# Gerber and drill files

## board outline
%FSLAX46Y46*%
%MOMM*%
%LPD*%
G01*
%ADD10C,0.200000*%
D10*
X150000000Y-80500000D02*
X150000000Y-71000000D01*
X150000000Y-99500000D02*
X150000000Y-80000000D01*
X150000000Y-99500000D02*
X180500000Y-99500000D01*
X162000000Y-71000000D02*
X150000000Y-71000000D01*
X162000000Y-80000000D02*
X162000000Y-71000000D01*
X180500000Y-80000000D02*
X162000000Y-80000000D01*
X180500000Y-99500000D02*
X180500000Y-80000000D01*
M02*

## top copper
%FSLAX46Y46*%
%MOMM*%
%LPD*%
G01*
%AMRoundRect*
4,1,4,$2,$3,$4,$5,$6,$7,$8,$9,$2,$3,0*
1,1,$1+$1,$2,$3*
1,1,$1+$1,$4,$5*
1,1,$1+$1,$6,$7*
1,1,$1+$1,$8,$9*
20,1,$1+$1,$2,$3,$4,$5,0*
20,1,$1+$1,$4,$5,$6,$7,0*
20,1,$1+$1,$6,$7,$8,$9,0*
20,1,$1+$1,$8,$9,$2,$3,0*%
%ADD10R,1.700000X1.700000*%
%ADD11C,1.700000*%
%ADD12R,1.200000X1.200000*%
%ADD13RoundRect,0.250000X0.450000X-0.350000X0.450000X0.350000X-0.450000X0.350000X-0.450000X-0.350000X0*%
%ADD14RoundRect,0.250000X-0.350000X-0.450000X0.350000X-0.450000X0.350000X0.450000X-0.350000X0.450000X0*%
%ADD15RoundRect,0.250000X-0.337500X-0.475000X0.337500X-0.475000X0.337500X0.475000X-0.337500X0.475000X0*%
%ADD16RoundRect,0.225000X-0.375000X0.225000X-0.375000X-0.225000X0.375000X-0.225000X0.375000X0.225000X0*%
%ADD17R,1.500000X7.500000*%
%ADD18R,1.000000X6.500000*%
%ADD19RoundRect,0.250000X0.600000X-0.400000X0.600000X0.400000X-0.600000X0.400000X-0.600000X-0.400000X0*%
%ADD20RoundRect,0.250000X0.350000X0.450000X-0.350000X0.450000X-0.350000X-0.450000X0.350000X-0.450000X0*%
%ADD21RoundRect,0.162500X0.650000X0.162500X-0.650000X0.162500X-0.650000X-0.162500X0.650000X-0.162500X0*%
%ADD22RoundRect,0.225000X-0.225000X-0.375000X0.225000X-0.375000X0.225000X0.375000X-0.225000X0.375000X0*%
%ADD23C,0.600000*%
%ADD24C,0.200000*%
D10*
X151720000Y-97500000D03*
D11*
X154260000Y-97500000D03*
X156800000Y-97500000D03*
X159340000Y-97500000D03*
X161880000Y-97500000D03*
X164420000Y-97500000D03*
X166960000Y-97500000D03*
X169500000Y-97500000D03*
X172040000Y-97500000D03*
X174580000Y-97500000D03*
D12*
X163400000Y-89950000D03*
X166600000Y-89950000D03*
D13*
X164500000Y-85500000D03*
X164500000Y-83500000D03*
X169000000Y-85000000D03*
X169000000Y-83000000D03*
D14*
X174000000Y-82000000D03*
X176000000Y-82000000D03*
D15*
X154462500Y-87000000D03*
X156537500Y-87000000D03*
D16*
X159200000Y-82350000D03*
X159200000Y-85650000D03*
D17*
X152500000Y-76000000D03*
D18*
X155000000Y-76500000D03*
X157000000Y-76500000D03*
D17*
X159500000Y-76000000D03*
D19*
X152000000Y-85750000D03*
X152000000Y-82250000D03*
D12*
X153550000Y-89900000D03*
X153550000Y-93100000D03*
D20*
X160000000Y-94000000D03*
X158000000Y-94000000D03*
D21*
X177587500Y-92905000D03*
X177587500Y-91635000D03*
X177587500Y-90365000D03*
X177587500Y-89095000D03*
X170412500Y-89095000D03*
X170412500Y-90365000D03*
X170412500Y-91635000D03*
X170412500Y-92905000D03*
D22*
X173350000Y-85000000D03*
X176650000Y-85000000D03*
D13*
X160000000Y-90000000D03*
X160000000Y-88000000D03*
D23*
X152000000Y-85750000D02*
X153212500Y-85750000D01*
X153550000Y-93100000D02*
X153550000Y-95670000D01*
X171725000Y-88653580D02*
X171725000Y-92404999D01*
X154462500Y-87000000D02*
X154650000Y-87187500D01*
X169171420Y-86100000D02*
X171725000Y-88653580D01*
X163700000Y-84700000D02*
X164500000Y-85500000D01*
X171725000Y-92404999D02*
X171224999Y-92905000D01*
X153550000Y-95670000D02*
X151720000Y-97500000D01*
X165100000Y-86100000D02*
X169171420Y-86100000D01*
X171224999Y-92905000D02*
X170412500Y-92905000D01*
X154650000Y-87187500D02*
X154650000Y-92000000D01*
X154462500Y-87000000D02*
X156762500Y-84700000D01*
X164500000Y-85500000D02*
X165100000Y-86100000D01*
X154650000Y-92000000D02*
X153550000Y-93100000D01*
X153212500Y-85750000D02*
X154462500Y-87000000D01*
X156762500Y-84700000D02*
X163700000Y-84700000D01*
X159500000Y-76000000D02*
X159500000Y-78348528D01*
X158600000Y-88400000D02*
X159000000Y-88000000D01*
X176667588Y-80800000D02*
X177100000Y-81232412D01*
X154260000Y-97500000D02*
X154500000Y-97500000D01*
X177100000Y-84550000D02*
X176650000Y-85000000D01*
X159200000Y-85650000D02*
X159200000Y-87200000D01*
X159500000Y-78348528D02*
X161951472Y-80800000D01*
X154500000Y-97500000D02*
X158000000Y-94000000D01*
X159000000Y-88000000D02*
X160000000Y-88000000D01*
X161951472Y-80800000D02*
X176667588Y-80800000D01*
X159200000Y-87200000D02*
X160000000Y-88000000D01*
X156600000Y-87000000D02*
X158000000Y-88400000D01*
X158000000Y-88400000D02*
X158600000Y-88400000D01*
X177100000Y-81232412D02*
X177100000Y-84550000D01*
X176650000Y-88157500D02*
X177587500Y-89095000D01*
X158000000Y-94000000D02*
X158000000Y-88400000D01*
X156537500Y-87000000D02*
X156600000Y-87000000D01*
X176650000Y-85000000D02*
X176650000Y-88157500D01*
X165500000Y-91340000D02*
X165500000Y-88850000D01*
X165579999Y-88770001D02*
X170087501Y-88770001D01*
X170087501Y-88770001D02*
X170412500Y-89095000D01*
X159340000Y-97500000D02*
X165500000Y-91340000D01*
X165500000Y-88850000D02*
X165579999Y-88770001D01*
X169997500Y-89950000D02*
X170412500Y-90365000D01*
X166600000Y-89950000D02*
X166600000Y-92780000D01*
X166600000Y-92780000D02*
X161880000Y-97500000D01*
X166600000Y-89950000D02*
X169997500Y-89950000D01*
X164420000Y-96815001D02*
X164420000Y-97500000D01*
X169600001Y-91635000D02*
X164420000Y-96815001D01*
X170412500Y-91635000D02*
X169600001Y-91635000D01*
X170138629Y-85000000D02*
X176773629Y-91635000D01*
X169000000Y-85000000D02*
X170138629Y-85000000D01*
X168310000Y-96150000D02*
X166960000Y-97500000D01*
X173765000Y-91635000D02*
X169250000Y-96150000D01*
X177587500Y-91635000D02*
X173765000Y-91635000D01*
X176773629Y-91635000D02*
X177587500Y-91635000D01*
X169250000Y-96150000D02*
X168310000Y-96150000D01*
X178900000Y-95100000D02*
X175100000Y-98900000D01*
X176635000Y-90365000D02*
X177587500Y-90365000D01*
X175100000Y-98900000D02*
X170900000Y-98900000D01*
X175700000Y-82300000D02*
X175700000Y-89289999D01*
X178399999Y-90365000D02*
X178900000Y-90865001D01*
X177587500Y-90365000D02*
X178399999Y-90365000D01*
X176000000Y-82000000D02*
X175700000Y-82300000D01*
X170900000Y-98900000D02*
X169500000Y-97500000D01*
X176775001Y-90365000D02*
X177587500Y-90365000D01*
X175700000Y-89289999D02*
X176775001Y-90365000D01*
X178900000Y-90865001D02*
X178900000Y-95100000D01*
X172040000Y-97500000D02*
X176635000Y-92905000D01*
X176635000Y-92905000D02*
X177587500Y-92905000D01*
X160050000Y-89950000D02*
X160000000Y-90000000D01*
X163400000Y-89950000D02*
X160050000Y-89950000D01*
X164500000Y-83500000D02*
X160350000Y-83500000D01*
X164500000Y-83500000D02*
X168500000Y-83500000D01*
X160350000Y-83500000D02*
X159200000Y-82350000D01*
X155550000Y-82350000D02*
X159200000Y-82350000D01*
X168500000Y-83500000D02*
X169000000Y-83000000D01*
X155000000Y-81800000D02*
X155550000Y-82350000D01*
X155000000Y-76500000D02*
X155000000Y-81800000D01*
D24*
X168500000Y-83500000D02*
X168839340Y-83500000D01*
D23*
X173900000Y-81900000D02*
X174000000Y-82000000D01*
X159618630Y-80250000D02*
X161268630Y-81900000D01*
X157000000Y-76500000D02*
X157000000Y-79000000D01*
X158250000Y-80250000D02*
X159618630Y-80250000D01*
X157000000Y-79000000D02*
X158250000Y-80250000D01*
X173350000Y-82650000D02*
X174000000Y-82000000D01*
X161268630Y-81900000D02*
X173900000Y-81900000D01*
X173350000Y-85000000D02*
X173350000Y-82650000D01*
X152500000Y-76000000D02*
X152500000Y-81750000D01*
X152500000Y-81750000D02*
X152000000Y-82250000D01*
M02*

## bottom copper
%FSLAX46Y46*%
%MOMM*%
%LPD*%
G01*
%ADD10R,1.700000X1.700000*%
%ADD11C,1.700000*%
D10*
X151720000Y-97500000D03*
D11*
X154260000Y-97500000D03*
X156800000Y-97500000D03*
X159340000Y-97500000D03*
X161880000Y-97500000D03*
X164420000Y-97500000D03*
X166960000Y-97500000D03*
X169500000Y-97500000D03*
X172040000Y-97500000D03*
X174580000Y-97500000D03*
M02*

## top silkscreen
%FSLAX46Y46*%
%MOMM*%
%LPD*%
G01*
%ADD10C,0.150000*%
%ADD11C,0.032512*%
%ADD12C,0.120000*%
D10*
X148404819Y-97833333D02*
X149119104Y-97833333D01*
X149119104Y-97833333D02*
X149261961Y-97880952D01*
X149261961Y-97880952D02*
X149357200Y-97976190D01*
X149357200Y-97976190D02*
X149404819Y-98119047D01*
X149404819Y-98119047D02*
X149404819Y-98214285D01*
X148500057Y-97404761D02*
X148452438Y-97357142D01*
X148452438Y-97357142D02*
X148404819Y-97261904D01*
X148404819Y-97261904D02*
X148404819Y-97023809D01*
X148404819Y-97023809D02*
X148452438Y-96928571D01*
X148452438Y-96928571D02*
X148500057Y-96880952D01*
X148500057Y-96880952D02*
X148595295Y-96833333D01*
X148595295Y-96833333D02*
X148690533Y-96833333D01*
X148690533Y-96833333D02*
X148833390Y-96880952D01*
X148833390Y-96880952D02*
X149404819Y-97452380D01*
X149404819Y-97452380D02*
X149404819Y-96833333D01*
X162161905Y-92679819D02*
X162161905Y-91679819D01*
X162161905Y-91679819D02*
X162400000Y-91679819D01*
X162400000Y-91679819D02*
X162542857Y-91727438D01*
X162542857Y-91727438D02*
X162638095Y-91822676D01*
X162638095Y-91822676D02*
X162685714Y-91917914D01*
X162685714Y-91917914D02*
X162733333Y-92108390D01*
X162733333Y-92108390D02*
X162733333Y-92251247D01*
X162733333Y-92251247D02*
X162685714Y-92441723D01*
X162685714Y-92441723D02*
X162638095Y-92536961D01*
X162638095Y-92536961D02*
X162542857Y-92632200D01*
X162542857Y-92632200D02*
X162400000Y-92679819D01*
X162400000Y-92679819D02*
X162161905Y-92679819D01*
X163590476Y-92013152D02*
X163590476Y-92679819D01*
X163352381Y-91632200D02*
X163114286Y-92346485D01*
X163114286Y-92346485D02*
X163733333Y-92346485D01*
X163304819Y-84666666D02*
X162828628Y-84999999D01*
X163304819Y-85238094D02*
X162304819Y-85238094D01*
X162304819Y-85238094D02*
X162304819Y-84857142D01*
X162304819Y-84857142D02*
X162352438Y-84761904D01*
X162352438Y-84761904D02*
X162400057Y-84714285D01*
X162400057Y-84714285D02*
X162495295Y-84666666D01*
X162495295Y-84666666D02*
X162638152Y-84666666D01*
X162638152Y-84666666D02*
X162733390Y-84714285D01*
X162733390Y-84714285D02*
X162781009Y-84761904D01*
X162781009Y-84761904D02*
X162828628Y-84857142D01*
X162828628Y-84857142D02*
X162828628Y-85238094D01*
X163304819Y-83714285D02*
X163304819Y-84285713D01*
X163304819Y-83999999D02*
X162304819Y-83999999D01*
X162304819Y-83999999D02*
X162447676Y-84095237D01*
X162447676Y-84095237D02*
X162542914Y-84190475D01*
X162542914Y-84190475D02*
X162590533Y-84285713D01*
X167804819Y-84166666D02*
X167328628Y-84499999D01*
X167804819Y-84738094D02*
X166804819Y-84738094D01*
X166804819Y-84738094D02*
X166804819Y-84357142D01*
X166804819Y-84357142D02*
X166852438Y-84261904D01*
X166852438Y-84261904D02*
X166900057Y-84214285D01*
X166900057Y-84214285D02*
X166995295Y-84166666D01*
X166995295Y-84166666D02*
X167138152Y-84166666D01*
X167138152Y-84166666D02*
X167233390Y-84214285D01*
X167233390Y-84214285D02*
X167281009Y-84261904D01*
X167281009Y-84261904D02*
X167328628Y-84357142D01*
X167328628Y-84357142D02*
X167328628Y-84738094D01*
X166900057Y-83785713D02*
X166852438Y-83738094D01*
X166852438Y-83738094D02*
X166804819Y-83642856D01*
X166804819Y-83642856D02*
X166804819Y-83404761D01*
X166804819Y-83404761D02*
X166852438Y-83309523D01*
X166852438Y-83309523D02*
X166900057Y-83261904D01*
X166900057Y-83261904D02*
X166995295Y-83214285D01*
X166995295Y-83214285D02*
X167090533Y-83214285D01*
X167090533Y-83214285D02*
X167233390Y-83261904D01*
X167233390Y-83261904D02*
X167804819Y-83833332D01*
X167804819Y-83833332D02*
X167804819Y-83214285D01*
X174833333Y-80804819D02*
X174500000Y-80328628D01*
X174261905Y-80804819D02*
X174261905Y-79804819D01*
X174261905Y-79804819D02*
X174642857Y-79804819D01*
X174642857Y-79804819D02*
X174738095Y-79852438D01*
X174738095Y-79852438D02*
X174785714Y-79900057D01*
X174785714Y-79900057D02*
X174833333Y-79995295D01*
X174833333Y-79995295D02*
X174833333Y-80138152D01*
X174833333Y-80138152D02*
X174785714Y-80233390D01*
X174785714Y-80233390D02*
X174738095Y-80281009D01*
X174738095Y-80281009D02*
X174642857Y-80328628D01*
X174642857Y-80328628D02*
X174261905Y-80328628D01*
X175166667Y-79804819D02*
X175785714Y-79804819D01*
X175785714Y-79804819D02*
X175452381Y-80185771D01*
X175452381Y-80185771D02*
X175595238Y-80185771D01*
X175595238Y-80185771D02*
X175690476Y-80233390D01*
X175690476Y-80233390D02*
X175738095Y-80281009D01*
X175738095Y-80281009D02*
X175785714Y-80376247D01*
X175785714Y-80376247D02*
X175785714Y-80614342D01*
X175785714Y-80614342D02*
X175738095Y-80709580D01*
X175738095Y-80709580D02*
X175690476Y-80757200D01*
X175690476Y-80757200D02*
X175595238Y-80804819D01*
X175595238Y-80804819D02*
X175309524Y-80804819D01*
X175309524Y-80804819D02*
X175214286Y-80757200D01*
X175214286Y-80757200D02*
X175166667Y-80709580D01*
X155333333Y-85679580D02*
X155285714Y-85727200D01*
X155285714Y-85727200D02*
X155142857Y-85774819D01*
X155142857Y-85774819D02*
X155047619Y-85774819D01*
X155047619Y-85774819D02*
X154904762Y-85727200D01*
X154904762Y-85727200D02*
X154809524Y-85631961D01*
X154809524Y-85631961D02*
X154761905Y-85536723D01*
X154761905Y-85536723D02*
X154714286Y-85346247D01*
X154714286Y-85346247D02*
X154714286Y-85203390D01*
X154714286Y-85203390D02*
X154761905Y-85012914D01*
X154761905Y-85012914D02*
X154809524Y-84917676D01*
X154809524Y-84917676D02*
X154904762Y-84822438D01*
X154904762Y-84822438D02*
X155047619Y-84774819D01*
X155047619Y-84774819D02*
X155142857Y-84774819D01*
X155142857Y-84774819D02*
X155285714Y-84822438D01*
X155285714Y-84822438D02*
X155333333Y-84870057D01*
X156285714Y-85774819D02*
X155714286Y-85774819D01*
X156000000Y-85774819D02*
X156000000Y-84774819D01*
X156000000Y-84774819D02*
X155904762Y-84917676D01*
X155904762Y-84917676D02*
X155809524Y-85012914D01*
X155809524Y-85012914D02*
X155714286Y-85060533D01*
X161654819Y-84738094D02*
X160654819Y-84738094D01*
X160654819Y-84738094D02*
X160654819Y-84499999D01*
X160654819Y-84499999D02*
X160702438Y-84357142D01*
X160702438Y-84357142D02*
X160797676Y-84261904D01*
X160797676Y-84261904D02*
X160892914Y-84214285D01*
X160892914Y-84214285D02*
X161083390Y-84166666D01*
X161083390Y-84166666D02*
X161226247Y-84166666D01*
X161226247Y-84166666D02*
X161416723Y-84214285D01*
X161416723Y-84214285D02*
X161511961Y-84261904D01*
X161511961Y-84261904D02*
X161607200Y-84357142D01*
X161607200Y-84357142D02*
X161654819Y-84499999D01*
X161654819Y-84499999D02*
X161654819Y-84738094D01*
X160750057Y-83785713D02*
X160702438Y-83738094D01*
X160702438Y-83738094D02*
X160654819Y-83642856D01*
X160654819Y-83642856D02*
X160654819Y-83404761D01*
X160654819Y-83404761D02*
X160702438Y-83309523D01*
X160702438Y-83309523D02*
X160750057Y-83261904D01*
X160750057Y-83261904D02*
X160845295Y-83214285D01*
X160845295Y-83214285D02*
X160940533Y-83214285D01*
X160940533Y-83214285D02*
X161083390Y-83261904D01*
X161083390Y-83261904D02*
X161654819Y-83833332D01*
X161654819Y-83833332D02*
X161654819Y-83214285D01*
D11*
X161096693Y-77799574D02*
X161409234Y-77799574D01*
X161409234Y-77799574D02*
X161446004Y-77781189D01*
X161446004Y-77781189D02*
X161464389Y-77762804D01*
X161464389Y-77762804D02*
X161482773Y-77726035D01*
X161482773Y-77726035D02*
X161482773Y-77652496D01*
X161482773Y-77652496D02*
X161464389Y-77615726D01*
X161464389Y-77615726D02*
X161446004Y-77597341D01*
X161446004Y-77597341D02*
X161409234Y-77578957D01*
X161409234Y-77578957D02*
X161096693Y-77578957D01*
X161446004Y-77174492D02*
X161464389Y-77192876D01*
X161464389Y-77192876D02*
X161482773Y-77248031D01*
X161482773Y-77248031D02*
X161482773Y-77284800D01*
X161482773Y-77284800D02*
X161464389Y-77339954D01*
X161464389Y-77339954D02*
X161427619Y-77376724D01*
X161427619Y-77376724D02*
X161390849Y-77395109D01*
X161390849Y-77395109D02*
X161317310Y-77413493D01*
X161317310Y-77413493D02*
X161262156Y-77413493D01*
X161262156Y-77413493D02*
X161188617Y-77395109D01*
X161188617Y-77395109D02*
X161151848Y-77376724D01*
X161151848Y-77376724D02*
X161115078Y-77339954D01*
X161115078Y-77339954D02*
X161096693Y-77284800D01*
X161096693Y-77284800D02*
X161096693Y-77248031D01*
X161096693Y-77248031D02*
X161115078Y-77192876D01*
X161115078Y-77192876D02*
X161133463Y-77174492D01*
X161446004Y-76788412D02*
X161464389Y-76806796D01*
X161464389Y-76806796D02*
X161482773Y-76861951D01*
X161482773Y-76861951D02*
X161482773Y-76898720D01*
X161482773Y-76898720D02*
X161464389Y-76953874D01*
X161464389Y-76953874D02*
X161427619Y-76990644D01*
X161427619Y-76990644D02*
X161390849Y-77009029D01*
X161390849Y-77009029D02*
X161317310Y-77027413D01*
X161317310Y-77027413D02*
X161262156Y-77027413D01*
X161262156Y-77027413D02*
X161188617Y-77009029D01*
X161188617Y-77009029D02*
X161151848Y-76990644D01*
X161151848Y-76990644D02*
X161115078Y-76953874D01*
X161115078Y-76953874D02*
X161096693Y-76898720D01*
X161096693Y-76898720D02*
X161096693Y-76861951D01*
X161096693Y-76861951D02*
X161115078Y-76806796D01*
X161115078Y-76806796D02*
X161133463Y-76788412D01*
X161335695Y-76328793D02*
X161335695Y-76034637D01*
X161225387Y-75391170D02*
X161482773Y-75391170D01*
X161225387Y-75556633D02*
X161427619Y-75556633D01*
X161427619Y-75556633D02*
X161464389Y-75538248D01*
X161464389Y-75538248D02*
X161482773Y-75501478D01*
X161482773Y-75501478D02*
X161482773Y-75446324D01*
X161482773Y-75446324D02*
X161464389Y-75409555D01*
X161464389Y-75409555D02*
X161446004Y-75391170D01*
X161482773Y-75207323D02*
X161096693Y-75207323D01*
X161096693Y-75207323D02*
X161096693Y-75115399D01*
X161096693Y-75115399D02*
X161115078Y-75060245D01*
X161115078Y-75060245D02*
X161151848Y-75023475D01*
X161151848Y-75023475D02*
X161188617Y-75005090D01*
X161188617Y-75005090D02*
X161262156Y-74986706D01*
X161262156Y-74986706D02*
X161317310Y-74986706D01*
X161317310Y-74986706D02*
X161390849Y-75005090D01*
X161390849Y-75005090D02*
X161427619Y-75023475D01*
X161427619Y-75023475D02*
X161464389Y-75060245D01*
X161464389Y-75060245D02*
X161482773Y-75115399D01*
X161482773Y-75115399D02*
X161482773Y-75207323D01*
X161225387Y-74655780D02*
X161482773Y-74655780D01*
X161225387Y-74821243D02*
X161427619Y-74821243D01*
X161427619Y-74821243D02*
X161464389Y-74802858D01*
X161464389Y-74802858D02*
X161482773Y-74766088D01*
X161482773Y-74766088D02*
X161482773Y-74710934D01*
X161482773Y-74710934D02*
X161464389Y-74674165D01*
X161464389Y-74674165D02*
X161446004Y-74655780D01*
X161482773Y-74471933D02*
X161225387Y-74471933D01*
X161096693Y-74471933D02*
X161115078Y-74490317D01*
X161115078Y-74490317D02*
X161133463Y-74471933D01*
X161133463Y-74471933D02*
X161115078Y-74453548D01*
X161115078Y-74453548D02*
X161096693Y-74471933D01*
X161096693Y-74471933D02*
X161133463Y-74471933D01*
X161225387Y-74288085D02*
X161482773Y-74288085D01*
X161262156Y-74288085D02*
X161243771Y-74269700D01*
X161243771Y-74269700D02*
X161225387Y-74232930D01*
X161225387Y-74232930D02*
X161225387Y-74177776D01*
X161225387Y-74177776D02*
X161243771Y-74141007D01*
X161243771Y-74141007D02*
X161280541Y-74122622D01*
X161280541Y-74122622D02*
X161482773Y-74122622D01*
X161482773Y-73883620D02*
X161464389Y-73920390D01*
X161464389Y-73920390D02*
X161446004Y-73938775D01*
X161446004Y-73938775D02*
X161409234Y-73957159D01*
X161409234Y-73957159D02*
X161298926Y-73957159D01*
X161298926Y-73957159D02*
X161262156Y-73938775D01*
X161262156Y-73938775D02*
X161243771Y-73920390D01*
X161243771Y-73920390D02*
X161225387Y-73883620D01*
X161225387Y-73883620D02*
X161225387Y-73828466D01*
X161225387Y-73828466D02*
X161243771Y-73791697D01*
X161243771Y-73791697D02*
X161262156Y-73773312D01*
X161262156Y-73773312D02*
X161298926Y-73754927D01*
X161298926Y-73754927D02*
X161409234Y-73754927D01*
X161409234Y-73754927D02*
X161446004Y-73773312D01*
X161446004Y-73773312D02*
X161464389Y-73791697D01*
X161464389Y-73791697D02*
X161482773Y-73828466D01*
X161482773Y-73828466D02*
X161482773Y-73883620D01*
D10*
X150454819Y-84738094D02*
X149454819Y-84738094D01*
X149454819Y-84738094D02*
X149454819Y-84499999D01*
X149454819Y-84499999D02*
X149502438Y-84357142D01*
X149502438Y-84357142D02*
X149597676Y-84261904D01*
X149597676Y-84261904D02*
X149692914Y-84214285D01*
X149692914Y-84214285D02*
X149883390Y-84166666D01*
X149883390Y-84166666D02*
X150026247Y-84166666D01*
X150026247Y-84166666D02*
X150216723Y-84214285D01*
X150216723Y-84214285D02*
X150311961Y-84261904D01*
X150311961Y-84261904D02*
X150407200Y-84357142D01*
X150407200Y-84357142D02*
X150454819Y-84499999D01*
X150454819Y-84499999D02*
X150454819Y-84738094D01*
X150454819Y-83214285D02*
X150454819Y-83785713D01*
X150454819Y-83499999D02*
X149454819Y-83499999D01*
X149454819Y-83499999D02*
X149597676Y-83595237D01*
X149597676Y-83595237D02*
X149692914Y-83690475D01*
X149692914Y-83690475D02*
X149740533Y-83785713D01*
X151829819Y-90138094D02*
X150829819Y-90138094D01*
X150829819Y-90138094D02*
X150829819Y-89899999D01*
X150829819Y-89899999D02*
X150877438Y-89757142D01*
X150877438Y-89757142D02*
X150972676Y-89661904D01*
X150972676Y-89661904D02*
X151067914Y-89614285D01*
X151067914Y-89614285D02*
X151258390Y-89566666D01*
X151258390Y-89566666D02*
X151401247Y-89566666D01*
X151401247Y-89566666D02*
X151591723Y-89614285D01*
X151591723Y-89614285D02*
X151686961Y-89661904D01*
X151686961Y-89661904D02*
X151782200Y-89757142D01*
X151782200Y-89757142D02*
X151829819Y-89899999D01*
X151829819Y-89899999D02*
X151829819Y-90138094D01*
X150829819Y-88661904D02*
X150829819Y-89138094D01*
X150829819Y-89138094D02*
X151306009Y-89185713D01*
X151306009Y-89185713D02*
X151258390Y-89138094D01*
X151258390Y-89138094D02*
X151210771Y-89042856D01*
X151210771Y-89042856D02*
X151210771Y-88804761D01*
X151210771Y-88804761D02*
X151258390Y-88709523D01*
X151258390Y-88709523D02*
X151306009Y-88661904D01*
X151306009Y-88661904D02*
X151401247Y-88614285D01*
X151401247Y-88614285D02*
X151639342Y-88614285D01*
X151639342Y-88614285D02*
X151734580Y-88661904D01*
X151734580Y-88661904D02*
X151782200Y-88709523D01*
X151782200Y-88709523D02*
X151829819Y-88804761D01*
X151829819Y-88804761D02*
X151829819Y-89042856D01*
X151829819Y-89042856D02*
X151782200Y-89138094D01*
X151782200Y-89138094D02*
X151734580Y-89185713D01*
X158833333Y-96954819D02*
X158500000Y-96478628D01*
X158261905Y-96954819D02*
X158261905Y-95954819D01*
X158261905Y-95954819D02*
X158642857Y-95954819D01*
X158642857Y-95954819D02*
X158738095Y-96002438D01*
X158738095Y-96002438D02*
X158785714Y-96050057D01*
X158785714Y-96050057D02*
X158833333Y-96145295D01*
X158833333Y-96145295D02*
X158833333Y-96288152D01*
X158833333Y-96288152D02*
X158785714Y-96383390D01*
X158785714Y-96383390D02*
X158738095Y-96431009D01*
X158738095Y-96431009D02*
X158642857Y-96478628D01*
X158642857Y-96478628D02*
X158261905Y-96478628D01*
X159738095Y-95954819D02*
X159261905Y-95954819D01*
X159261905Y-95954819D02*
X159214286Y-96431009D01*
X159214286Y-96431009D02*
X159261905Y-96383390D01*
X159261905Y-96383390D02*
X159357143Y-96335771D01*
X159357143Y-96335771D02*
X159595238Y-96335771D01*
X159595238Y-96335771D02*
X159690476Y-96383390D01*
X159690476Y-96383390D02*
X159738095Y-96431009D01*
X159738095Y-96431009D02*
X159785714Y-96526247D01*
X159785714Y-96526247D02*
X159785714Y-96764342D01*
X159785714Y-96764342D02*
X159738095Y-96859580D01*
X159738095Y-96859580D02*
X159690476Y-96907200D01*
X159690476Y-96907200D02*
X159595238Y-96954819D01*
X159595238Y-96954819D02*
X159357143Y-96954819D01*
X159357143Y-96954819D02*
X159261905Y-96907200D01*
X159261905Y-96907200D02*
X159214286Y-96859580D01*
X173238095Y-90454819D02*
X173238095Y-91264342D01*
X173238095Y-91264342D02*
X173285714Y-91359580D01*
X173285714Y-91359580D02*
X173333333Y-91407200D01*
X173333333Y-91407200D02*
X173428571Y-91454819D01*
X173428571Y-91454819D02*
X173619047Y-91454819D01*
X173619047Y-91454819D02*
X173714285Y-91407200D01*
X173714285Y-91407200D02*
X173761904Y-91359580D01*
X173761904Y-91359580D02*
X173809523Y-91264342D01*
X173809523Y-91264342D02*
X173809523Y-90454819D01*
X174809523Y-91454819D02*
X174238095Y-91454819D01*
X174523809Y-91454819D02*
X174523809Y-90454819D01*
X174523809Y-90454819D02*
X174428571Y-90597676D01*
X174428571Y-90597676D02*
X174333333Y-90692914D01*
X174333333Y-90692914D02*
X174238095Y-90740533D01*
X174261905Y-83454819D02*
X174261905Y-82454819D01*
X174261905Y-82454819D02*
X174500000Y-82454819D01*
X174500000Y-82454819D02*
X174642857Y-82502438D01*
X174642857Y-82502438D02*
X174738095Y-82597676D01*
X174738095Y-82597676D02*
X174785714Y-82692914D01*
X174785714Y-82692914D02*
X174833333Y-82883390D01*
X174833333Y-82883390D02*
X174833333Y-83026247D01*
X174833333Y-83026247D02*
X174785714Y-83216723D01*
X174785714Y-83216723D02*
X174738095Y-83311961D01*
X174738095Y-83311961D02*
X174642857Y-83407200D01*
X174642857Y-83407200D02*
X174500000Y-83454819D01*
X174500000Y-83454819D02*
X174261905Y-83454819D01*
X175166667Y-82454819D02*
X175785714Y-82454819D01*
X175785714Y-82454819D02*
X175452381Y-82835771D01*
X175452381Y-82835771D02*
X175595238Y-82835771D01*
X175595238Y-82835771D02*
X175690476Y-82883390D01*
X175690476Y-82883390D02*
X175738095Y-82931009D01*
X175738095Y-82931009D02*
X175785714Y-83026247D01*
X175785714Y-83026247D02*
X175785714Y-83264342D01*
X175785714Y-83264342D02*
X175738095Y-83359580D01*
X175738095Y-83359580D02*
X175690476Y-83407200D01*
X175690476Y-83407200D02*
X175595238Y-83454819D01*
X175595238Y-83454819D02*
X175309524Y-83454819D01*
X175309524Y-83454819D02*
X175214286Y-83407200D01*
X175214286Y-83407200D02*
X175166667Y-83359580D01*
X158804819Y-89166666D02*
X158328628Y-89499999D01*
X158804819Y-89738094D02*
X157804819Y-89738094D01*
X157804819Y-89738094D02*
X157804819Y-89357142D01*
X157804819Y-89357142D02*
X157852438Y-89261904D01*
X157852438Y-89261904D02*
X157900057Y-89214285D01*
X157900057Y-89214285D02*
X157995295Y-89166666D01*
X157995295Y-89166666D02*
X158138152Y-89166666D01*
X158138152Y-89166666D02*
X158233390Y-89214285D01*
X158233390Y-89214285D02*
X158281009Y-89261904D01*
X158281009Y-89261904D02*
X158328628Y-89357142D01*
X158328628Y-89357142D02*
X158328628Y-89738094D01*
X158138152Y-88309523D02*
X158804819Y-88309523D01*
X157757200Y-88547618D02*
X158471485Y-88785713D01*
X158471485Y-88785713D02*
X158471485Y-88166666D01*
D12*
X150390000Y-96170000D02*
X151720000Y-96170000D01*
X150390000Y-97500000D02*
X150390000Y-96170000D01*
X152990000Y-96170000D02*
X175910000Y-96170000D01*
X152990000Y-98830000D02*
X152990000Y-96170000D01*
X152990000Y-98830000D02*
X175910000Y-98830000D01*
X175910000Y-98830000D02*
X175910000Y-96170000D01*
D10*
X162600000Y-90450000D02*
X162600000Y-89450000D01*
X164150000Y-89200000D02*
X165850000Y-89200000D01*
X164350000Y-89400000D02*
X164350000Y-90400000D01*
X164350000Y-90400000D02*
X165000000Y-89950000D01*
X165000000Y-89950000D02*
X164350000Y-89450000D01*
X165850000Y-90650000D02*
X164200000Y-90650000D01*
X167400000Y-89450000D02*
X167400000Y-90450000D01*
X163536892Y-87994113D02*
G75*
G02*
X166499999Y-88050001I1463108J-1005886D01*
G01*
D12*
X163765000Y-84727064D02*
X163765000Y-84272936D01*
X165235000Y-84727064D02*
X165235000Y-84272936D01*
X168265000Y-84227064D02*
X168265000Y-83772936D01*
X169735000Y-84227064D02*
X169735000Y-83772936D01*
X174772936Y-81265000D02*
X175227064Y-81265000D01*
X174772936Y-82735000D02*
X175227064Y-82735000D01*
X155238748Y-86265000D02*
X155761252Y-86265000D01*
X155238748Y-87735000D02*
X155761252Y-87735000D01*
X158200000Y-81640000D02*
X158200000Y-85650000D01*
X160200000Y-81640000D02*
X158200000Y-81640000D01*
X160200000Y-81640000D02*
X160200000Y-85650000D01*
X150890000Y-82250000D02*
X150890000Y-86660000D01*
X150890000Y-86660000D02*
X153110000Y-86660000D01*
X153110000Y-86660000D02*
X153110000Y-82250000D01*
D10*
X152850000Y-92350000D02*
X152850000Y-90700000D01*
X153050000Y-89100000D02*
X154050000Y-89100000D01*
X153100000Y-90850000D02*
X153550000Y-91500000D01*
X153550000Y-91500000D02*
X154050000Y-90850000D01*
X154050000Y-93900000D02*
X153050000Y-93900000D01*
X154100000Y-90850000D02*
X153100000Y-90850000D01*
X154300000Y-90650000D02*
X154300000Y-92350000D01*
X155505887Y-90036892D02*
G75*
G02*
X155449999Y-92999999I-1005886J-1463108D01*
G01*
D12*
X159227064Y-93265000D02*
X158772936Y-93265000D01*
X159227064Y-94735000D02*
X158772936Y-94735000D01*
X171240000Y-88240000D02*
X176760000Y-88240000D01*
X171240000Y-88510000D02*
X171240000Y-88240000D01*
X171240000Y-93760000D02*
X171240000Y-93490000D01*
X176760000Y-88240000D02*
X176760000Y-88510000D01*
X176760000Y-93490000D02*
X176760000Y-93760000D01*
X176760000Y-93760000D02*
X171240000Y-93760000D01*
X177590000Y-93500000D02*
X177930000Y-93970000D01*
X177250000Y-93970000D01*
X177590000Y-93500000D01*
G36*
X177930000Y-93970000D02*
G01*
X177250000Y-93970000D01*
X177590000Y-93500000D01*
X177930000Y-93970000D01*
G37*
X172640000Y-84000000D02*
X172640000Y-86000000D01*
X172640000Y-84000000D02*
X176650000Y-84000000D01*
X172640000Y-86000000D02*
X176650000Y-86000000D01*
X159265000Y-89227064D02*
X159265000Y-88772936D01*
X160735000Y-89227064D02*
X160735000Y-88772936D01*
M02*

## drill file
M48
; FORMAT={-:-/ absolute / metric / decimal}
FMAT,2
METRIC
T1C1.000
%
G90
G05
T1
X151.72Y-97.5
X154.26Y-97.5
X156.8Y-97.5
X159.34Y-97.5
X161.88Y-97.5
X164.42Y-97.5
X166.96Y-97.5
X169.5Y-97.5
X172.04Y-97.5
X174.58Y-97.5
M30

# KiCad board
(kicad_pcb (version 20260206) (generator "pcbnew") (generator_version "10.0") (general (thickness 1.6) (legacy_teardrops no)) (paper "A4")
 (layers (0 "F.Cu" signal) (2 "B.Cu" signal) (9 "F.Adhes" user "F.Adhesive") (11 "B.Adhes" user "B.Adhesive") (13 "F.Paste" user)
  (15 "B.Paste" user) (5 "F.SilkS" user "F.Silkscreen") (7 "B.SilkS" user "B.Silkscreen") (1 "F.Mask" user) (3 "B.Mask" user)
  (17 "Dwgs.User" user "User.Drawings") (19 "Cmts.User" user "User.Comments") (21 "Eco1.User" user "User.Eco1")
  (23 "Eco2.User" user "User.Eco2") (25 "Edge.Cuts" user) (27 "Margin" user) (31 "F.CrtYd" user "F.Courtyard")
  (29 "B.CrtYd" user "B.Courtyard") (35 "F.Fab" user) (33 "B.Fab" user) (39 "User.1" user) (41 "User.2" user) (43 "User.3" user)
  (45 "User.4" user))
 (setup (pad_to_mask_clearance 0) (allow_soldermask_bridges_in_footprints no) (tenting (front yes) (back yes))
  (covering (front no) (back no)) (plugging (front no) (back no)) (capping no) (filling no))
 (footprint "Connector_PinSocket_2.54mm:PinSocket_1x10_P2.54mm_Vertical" (layer "F.Cu") (at 151.72 97.5 90)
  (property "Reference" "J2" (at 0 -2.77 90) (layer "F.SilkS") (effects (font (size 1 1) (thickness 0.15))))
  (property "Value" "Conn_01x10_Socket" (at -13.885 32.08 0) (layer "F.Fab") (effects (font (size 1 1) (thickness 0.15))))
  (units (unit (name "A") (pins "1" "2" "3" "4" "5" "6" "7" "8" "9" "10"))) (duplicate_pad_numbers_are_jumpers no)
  (fp_line (start 1.33 -1.33) (end 1.33 0) (stroke (width 0.12) (type solid)) (layer "F.SilkS"))
  (fp_line (start 0 -1.33) (end 1.33 -1.33) (stroke (width 0.12) (type solid)) (layer "F.SilkS"))
  (fp_line (start 1.33 1.27) (end 1.33 24.19) (stroke (width 0.12) (type solid)) (layer "F.SilkS"))
  (fp_line (start -1.33 1.27) (end 1.33 1.27) (stroke (width 0.12) (type solid)) (layer "F.SilkS"))
  (fp_line (start -1.33 1.27) (end -1.33 24.19) (stroke (width 0.12) (type solid)) (layer "F.SilkS"))
  (fp_line (start -1.33 24.19) (end 1.33 24.19) (stroke (width 0.12) (type solid)) (layer "F.SilkS"))
  (pad "1" thru_hole rect (at 0 0 90) (size 1.7 1.7) (drill 1) (layers "*.Cu" "*.Mask") (remove_unused_layers no) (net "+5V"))
  (pad "2" thru_hole circle (at 0 2.54 90) (size 1.7 1.7) (drill 1) (layers "*.Cu" "*.Mask") (remove_unused_layers no) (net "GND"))
  (pad "3" thru_hole circle (at 0 5.08 90) (size 1.7 1.7) (drill 1) (layers "*.Cu" "*.Mask") (remove_unused_layers no)
   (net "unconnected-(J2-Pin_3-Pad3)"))
  (pad "4" thru_hole circle (at 0 7.62 90) (size 1.7 1.7) (drill 1) (layers "*.Cu" "*.Mask") (remove_unused_layers no)
   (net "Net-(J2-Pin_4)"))
  (pad "5" thru_hole circle (at 0 10.16 90) (size 1.7 1.7) (drill 1) (layers "*.Cu" "*.Mask") (remove_unused_layers no) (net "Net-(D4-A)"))
  (pad "6" thru_hole circle (at 0 12.7 90) (size 1.7 1.7) (drill 1) (layers "*.Cu" "*.Mask") (remove_unused_layers no)
   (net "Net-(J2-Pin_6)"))
  (pad "7" thru_hole circle (at 0 15.24 90) (size 1.7 1.7) (drill 1) (layers "*.Cu" "*.Mask") (remove_unused_layers no)
   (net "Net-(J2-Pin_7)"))
  (pad "8" thru_hole circle (at 0 17.78 90) (size 1.7 1.7) (drill 1) (layers "*.Cu" "*.Mask") (remove_unused_layers no)
   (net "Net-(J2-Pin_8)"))
  (pad "9" thru_hole circle (at 0 20.32 90) (size 1.7 1.7) (drill 1) (layers "*.Cu" "*.Mask") (remove_unused_layers no)
   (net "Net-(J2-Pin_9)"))
  (pad "10" thru_hole circle (at 0 22.86 90) (size 1.7 1.7) (drill 1) (layers "*.Cu" "*.Mask") (remove_unused_layers no)
   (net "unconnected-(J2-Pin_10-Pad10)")))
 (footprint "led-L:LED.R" (layer "F.Cu") (at 165.5 89.5)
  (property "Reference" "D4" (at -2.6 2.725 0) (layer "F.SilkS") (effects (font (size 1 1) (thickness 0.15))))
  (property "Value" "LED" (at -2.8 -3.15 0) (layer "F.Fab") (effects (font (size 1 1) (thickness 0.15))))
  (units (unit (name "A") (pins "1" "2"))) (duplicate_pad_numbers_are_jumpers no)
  (fp_line (start -2.9 0.95) (end -2.9 -0.05) (stroke (width 0.15) (type solid)) (layer "F.SilkS"))
  (fp_line (start -1.35 -0.3) (end 0.35 -0.3) (stroke (width 0.15) (type solid)) (layer "F.SilkS"))
  (fp_line (start -1.15 -0.1) (end -1.15 0.9) (stroke (width 0.15) (type solid)) (layer "F.SilkS"))
  (fp_line (start -1.15 0.9) (end -0.5 0.45) (stroke (width 0.15) (type solid)) (layer "F.SilkS"))
  (fp_line (start -0.5 0.45) (end -1.15 -0.05) (stroke (width 0.15) (type solid)) (layer "F.SilkS"))
  (fp_line (start 0.35 1.15) (end -1.3 1.15) (stroke (width 0.15) (type solid)) (layer "F.SilkS"))
  (fp_line (start 1.9 -0.05) (end 1.9 0.95) (stroke (width 0.15) (type solid)) (layer "F.SilkS"))
  (fp_arc (start -1.963108 -1.505887) (mid -0.466517 -2.275211) (end 0.999999 -1.449999) (stroke (width 0.15) (type solid))
   (layer "F.SilkS"))
  (pad "1" smd rect (at -2.1 0.45) (size 1.2 1.2) (layers "F.Cu" "F.Mask" "F.Paste") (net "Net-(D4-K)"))
  (pad "2" smd rect (at 1.1 0.45) (size 1.2 1.2) (layers "F.Cu" "F.Mask" "F.Paste") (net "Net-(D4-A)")))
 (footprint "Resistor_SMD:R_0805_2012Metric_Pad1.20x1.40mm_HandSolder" (layer "F.Cu") (at 164.5 84.5 90)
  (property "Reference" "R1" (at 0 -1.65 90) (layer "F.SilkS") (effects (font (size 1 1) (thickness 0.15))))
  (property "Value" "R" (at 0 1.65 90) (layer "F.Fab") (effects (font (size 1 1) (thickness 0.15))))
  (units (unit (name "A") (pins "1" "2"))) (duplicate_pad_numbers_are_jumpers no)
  (fp_line (start -0.227064 -0.735) (end 0.227064 -0.735) (stroke (width 0.12) (type solid)) (layer "F.SilkS"))
  (fp_line (start -0.227064 0.735) (end 0.227064 0.735) (stroke (width 0.12) (type solid)) (layer "F.SilkS"))
  (pad "1" smd roundrect (at -1 0 90) (size 1.2 1.4) (layers "F.Cu" "F.Mask" "F.Paste") (roundrect_rratio 0.208333) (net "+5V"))
  (pad "2" smd roundrect (at 1 0 90) (size 1.2 1.4) (layers "F.Cu" "F.Mask" "F.Paste") (roundrect_rratio 0.208333) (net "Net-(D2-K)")))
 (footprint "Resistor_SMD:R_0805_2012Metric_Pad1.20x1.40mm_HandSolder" (layer "F.Cu") (at 169 84 90)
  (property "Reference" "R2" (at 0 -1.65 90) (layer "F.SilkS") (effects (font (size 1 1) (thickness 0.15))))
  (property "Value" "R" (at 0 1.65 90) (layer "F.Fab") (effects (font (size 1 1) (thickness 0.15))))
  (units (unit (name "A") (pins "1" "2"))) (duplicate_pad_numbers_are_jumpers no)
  (fp_line (start -0.227064 -0.735) (end 0.227064 -0.735) (stroke (width 0.12) (type solid)) (layer "F.SilkS"))
  (fp_line (start -0.227064 0.735) (end 0.227064 0.735) (stroke (width 0.12) (type solid)) (layer "F.SilkS"))
  (pad "1" smd roundrect (at -1 0 90) (size 1.2 1.4) (layers "F.Cu" "F.Mask" "F.Paste") (roundrect_rratio 0.208333) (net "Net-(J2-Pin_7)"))
  (pad "2" smd roundrect (at 1 0 90) (size 1.2 1.4) (layers "F.Cu" "F.Mask" "F.Paste") (roundrect_rratio 0.208333) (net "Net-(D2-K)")))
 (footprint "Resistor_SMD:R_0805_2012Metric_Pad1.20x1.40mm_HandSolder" (layer "F.Cu") (at 175 82)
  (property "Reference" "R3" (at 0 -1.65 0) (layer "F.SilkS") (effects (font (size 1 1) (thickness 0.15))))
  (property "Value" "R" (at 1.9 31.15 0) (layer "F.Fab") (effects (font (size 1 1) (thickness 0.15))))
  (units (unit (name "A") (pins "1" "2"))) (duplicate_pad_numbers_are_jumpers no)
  (fp_line (start -0.227064 -0.735) (end 0.227064 -0.735) (stroke (width 0.12) (type solid)) (layer "F.SilkS"))
  (fp_line (start -0.227064 0.735) (end 0.227064 0.735) (stroke (width 0.12) (type solid)) (layer "F.SilkS"))
  (pad "1" smd roundrect (at -1 0) (size 1.2 1.4) (layers "F.Cu" "F.Mask" "F.Paste") (roundrect_rratio 0.208333) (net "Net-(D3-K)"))
  (pad "2" smd roundrect (at 1 0) (size 1.2 1.4) (layers "F.Cu" "F.Mask" "F.Paste") (roundrect_rratio 0.208333) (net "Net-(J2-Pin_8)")))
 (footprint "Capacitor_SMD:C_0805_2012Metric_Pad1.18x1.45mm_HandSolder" (layer "F.Cu") (at 155.5 87)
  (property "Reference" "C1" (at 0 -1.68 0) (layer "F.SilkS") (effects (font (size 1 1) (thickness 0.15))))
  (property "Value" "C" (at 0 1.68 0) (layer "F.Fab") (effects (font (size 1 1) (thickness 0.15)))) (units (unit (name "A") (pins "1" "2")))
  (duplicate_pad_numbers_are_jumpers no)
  (fp_line (start -0.261252 -0.735) (end 0.261252 -0.735) (stroke (width 0.12) (type solid)) (layer "F.SilkS"))
  (fp_line (start -0.261252 0.735) (end 0.261252 0.735) (stroke (width 0.12) (type solid)) (layer "F.SilkS"))
  (pad "1" smd roundrect (at -1.0375 0) (size 1.175 1.45) (layers "F.Cu" "F.Mask" "F.Paste") (roundrect_rratio 0.212766) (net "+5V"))
  (pad "2" smd roundrect (at 1.0375 0) (size 1.175 1.45) (layers "F.Cu" "F.Mask" "F.Paste") (roundrect_rratio 0.212766) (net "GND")))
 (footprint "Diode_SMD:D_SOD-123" (layer "F.Cu") (at 159.2 84 -90)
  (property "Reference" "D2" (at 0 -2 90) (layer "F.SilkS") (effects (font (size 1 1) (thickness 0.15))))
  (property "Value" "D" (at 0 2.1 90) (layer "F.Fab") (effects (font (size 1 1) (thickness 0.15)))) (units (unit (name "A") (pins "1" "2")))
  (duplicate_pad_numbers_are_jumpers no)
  (fp_line (start -2.36 1) (end 1.65 1) (stroke (width 0.12) (type solid)) (layer "F.SilkS"))
  (fp_line (start -2.36 -1) (end -2.36 1) (stroke (width 0.12) (type solid)) (layer "F.SilkS"))
  (fp_line (start -2.36 -1) (end 1.65 -1) (stroke (width 0.12) (type solid)) (layer "F.SilkS"))
  (pad "1" smd roundrect (at -1.65 0 270) (size 0.9 1.2) (layers "F.Cu" "F.Mask" "F.Paste") (roundrect_rratio 0.25) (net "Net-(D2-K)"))
  (pad "2" smd roundrect (at 1.65 0 270) (size 0.9 1.2) (layers "F.Cu" "F.Mask" "F.Paste") (roundrect_rratio 0.25) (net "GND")))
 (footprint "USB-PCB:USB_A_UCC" (layer "F.Cu") (at 156 76.2 -90)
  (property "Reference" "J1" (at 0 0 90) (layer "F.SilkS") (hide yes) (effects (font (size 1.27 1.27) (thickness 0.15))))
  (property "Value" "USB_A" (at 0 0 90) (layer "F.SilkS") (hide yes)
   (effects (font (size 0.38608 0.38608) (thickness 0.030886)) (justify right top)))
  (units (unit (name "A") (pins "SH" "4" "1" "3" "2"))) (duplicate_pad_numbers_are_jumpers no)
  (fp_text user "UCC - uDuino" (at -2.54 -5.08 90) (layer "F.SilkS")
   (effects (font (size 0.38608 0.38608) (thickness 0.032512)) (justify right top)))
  (pad "1" smd rect (at -0.2 3.5 270) (size 7.5 1.5) (layers "F.Cu" "F.Mask" "F.Paste") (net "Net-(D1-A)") (solder_mask_margin 0.1016))
  (pad "2" smd rect (at 0.3 1 270) (size 6.5 1) (layers "F.Cu" "F.Mask" "F.Paste") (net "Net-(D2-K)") (solder_mask_margin 0.1016))
  (pad "3" smd rect (at 0.3 -1 270) (size 6.5 1) (layers "F.Cu" "F.Mask" "F.Paste") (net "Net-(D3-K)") (solder_mask_margin 0.1016))
  (pad "4" smd rect (at -0.2 -3.5 270) (size 7.5 1.5) (layers "F.Cu" "F.Mask" "F.Paste") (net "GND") (solder_mask_margin 0.1016)))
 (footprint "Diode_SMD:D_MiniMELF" (layer "F.Cu") (at 152 84 90)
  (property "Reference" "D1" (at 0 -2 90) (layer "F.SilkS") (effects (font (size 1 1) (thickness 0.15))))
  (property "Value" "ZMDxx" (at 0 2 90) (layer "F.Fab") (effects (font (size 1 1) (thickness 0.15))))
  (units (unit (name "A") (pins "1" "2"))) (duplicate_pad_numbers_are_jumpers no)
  (fp_line (start 1.75 -1.11) (end -2.66 -1.11) (stroke (width 0.12) (type solid)) (layer "F.SilkS"))
  (fp_line (start -2.66 -1.11) (end -2.66 1.11) (stroke (width 0.12) (type solid)) (layer "F.SilkS"))
  (fp_line (start -2.66 1.11) (end 1.75 1.11) (stroke (width 0.12) (type solid)) (layer "F.SilkS"))
  (pad "1" smd roundrect (at -1.75 0 90) (size 1.3 1.7) (layers "F.Cu" "F.Mask" "F.Paste") (roundrect_rratio 0.1923076923) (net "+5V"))
  (pad "2" smd roundrect (at 1.75 0 90) (size 1.3 1.7) (layers "F.Cu" "F.Mask" "F.Paste") (roundrect_rratio 0.1923076923) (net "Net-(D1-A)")))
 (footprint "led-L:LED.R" (layer "F.Cu") (at 154 92 -90)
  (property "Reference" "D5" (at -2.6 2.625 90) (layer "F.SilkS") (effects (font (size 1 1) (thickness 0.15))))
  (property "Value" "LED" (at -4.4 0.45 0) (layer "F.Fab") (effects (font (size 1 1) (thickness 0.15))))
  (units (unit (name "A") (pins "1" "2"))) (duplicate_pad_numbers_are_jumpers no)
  (fp_line (start 0.35 1.15) (end -1.3 1.15) (stroke (width 0.15) (type solid)) (layer "F.SilkS"))
  (fp_line (start -2.9 0.95) (end -2.9 -0.05) (stroke (width 0.15) (type solid)) (layer "F.SilkS"))
  (fp_line (start -1.15 0.9) (end -0.5 0.45) (stroke (width 0.15) (type solid)) (layer "F.SilkS"))
  (fp_line (start -0.5 0.45) (end -1.15 -0.05) (stroke (width 0.15) (type solid)) (layer "F.SilkS"))
  (fp_line (start 1.9 -0.05) (end 1.9 0.95) (stroke (width 0.15) (type solid)) (layer "F.SilkS"))
  (fp_line (start -1.15 -0.1) (end -1.15 0.9) (stroke (width 0.15) (type solid)) (layer "F.SilkS"))
  (fp_line (start -1.35 -0.3) (end 0.35 -0.3) (stroke (width 0.15) (type solid)) (layer "F.SilkS"))
  (fp_arc (start -1.963108 -1.505887) (mid -0.466517 -2.275211) (end 0.999999 -1.449999) (stroke (width 0.15) (type solid))
   (layer "F.SilkS"))
  (pad "1" smd rect (at -2.1 0.45 270) (size 1.2 1.2) (layers "F.Cu" "F.Mask" "F.Paste") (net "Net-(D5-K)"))
  (pad "2" smd rect (at 1.1 0.45 270) (size 1.2 1.2) (layers "F.Cu" "F.Mask" "F.Paste") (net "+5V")))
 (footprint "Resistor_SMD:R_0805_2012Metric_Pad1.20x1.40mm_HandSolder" (layer "F.Cu") (at 159 94 180)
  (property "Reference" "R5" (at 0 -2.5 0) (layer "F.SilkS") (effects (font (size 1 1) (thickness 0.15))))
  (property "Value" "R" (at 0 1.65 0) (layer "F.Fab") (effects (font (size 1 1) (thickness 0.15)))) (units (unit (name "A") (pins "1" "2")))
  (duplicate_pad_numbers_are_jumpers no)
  (fp_line (start -0.227064 0.735) (end 0.227064 0.735) (stroke (width 0.12) (type solid)) (layer "F.SilkS"))
  (fp_line (start -0.227064 -0.735) (end 0.227064 -0.735) (stroke (width 0.12) (type solid)) (layer "F.SilkS"))
  (pad "1" smd roundrect (at -1 0 180) (size 1.2 1.4) (layers "F.Cu" "F.Mask" "F.Paste") (roundrect_rratio 0.208333) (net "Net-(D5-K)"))
  (pad "2" smd roundrect (at 1 0 180) (size 1.2 1.4) (layers "F.Cu" "F.Mask" "F.Paste") (roundrect_rratio 0.208333) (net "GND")))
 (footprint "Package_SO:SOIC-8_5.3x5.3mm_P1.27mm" (layer "F.Cu") (at 174 91 180)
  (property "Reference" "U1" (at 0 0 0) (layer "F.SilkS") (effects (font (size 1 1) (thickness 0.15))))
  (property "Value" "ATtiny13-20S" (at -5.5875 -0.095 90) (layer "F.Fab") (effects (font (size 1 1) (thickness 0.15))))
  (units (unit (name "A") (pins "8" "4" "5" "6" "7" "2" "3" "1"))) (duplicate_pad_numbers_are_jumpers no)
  (fp_line (start 2.76 2.76) (end -2.76 2.76) (stroke (width 0.12) (type solid)) (layer "F.SilkS"))
  (fp_line (start 2.76 2.49) (end 2.76 2.76) (stroke (width 0.12) (type solid)) (layer "F.SilkS"))
  (fp_line (start 2.76 -2.76) (end 2.76 -2.49) (stroke (width 0.12) (type solid)) (layer "F.SilkS"))
  (fp_line (start -2.76 2.76) (end -2.76 2.49) (stroke (width 0.12) (type solid)) (layer "F.SilkS"))
  (fp_line (start -2.76 -2.49) (end -2.76 -2.76) (stroke (width 0.12) (type solid)) (layer "F.SilkS"))
  (fp_line (start -2.76 -2.76) (end 2.76 -2.76) (stroke (width 0.12) (type solid)) (layer "F.SilkS"))
  (fp_poly (pts (xy -3.59 -2.5) (xy -3.93 -2.97) (xy -3.25 -2.97)) (stroke (width 0.12) (type solid)) (fill yes) (layer "F.SilkS"))
  (pad "1" smd roundrect (at -3.5875 -1.905 180) (size 1.625 0.65) (layers "F.Cu" "F.Mask" "F.Paste") (roundrect_rratio 0.25)
   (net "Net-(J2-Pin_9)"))
  (pad "2" smd roundrect (at -3.5875 -0.635 180) (size 1.625 0.65) (layers "F.Cu" "F.Mask" "F.Paste") (roundrect_rratio 0.25)
   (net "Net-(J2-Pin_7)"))
  (pad "3" smd roundrect (at -3.5875 0.635 180) (size 1.625 0.65) (layers "F.Cu" "F.Mask" "F.Paste") (roundrect_rratio 0.25)
   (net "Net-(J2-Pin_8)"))
  (pad "4" smd roundrect (at -3.5875 1.905 180) (size 1.625 0.65) (layers "F.Cu" "F.Mask" "F.Paste") (roundrect_rratio 0.25) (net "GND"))
  (pad "5" smd roundrect (at 3.5875 1.905 180) (size 1.625 0.65) (layers "F.Cu" "F.Mask" "F.Paste") (roundrect_rratio 0.25)
   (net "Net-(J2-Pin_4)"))
  (pad "6" smd roundrect (at 3.5875 0.635 180) (size 1.625 0.65) (layers "F.Cu" "F.Mask" "F.Paste") (roundrect_rratio 0.25)
   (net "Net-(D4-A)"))
  (pad "7" smd roundrect (at 3.5875 -0.635 180) (size 1.625 0.65) (layers "F.Cu" "F.Mask" "F.Paste") (roundrect_rratio 0.25)
   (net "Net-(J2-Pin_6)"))
  (pad "8" smd roundrect (at 3.5875 -1.905 180) (size 1.625 0.65) (layers "F.Cu" "F.Mask" "F.Paste") (roundrect_rratio 0.25) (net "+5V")))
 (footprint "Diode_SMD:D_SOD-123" (layer "F.Cu") (at 175 85)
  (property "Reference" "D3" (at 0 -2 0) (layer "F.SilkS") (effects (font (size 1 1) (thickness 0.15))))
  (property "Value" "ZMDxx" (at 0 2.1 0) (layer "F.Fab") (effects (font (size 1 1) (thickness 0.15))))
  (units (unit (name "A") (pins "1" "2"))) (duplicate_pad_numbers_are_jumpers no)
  (fp_line (start -2.36 -1) (end -2.36 1) (stroke (width 0.12) (type solid)) (layer "F.SilkS"))
  (fp_line (start -2.36 -1) (end 1.65 -1) (stroke (width 0.12) (type solid)) (layer "F.SilkS"))
  (fp_line (start -2.36 1) (end 1.65 1) (stroke (width 0.12) (type solid)) (layer "F.SilkS"))
  (pad "1" smd roundrect (at -1.65 0) (size 0.9 1.2) (layers "F.Cu" "F.Mask" "F.Paste") (roundrect_rratio 0.25) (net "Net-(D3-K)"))
  (pad "2" smd roundrect (at 1.65 0) (size 0.9 1.2) (layers "F.Cu" "F.Mask" "F.Paste") (roundrect_rratio 0.25) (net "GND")))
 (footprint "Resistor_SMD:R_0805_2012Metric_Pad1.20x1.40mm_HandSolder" (layer "F.Cu") (at 160 89 90)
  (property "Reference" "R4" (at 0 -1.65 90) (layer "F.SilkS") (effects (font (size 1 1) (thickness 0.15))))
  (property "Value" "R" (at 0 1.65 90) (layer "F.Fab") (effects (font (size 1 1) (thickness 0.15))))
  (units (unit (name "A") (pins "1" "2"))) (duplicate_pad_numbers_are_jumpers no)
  (fp_line (start -0.227064 -0.735) (end 0.227064 -0.735) (stroke (width 0.12) (type solid)) (layer "F.SilkS"))
  (fp_line (start -0.227064 0.735) (end 0.227064 0.735) (stroke (width 0.12) (type solid)) (layer "F.SilkS"))
  (pad "1" smd roundrect (at -1 0 90) (size 1.2 1.4) (layers "F.Cu" "F.Mask" "F.Paste") (roundrect_rratio 0.208333) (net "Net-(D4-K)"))
  (pad "2" smd roundrect (at 1 0 90) (size 1.2 1.4) (layers "F.Cu" "F.Mask" "F.Paste") (roundrect_rratio 0.208333) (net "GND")))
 (gr_line (start 150 80.5) (end 150 71) (stroke (width 0.2) (type solid)) (layer "Edge.Cuts"))
 (gr_line (start 150 99.5) (end 150 80) (stroke (width 0.2) (type solid)) (layer "Edge.Cuts"))
 (gr_line (start 150 99.5) (end 180.5 99.5) (stroke (width 0.2) (type solid)) (layer "Edge.Cuts"))
 (gr_line (start 162 71) (end 150 71) (stroke (width 0.2) (type solid)) (layer "Edge.Cuts"))
 (gr_line (start 162 80) (end 162 71) (stroke (width 0.2) (type solid)) (layer "Edge.Cuts"))
 (gr_line (start 180.5 80) (end 162 80) (stroke (width 0.2) (type solid)) (layer "Edge.Cuts"))
 (gr_line (start 180.5 99.5) (end 180.5 80) (stroke (width 0.2) (type solid)) (layer "Edge.Cuts"))
 (segment (start 152 85.75) (end 153.2125 85.75) (width 0.6) (layer "F.Cu") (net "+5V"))
 (segment (start 153.55 93.1) (end 153.55 95.67) (width 0.6) (layer "F.Cu") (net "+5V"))
 (segment (start 171.725 88.65358) (end 171.725 92.404999) (width 0.6) (layer "F.Cu") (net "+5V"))
 (segment (start 154.4625 87) (end 154.65 87.1875) (width 0.6) (layer "F.Cu") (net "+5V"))
 (segment (start 169.17142 86.1) (end 171.725 88.65358) (width 0.6) (layer "F.Cu") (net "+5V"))
 (segment (start 163.7 84.7) (end 164.5 85.5) (width 0.6) (layer "F.Cu") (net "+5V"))
 (segment (start 171.725 92.404999) (end 171.224999 92.905) (width 0.6) (layer "F.Cu") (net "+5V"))
 (segment (start 153.55 95.67) (end 151.72 97.5) (width 0.6) (layer "F.Cu") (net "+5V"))
 (segment (start 165.1 86.1) (end 169.17142 86.1) (width 0.6) (layer "F.Cu") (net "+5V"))
 (segment (start 171.224999 92.905) (end 170.4125 92.905) (width 0.6) (layer "F.Cu") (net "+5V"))
 (segment (start 154.65 87.1875) (end 154.65 92) (width 0.6) (layer "F.Cu") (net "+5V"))
 (segment (start 154.4625 87) (end 156.7625 84.7) (width 0.6) (layer "F.Cu") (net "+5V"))
 (segment (start 164.5 85.5) (end 165.1 86.1) (width 0.6) (layer "F.Cu") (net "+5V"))
 (segment (start 154.65 92) (end 153.55 93.1) (width 0.6) (layer "F.Cu") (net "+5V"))
 (segment (start 153.2125 85.75) (end 154.4625 87) (width 0.6) (layer "F.Cu") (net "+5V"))
 (segment (start 156.7625 84.7) (end 163.7 84.7) (width 0.6) (layer "F.Cu") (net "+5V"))
 (segment (start 159.5 76) (end 159.5 78.348528) (width 0.6) (layer "F.Cu") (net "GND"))
 (segment (start 158.6 88.4) (end 159 88) (width 0.6) (layer "F.Cu") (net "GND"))
 (segment (start 176.667588 80.8) (end 177.1 81.232412) (width 0.6) (layer "F.Cu") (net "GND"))
 (segment (start 154.26 97.5) (end 154.5 97.5) (width 0.6) (layer "F.Cu") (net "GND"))
 (segment (start 177.1 84.55) (end 176.65 85) (width 0.6) (layer "F.Cu") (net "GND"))
 (segment (start 159.2 85.65) (end 159.2 87.2) (width 0.6) (layer "F.Cu") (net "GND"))
 (segment (start 159.5 78.348528) (end 161.951472 80.8) (width 0.6) (layer "F.Cu") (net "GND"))
 (segment (start 154.5 97.5) (end 158 94) (width 0.6) (layer "F.Cu") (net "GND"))
 (segment (start 159 88) (end 160 88) (width 0.6) (layer "F.Cu") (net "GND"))
 (segment (start 161.951472 80.8) (end 176.667588 80.8) (width 0.6) (layer "F.Cu") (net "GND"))
 (segment (start 159.2 87.2) (end 160 88) (width 0.6) (layer "F.Cu") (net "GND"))
 (segment (start 156.6 87) (end 158 88.4) (width 0.6) (layer "F.Cu") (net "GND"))
 (segment (start 158 88.4) (end 158.6 88.4) (width 0.6) (layer "F.Cu") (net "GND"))
 (segment (start 177.1 81.232412) (end 177.1 84.55) (width 0.6) (layer "F.Cu") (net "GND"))
 (segment (start 176.65 88.1575) (end 177.5875 89.095) (width 0.6) (layer "F.Cu") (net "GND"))
 (segment (start 158 94) (end 158 88.4) (width 0.6) (layer "F.Cu") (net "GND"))
 (segment (start 156.5375 87) (end 156.6 87) (width 0.6) (layer "F.Cu") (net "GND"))
 (segment (start 176.65 85) (end 176.65 88.1575) (width 0.6) (layer "F.Cu") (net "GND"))
 (segment (start 165.5 91.34) (end 165.5 88.85) (width 0.6) (layer "F.Cu") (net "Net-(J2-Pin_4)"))
 (segment (start 165.579999 88.770001) (end 170.087501 88.770001) (width 0.6) (layer "F.Cu") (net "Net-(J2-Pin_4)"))
 (segment (start 170.087501 88.770001) (end 170.4125 89.095) (width 0.6) (layer "F.Cu") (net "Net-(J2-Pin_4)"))
 (segment (start 159.34 97.5) (end 165.5 91.34) (width 0.6) (layer "F.Cu") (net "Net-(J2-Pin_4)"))
 (segment (start 165.5 88.85) (end 165.579999 88.770001) (width 0.6) (layer "F.Cu") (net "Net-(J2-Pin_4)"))
 (segment (start 169.9975 89.95) (end 170.4125 90.365) (width 0.6) (layer "F.Cu") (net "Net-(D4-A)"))
 (segment (start 166.6 89.95) (end 166.6 92.78) (width 0.6) (layer "F.Cu") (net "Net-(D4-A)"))
 (segment (start 166.6 92.78) (end 161.88 97.5) (width 0.6) (layer "F.Cu") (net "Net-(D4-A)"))
 (segment (start 166.6 89.95) (end 169.9975 89.95) (width 0.6) (layer "F.Cu") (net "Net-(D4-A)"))
 (segment (start 164.42 96.815001) (end 164.42 97.5) (width 0.6) (layer "F.Cu") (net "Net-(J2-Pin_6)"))
 (segment (start 169.600001 91.635) (end 164.42 96.815001) (width 0.6) (layer "F.Cu") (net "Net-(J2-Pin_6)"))
 (segment (start 170.4125 91.635) (end 169.600001 91.635) (width 0.6) (layer "F.Cu") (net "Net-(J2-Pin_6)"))
 (segment (start 170.138629 85) (end 176.773629 91.635) (width 0.6) (layer "F.Cu") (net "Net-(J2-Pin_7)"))
 (segment (start 169 85) (end 170.138629 85) (width 0.6) (layer "F.Cu") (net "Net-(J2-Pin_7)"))
 (segment (start 168.31 96.15) (end 166.96 97.5) (width 0.6) (layer "F.Cu") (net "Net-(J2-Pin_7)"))
 (segment (start 173.765 91.635) (end 169.25 96.15) (width 0.6) (layer "F.Cu") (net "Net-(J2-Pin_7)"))
 (segment (start 177.5875 91.635) (end 173.765 91.635) (width 0.6) (layer "F.Cu") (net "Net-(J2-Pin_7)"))
 (segment (start 176.773629 91.635) (end 177.5875 91.635) (width 0.6) (layer "F.Cu") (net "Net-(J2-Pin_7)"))
 (segment (start 169.25 96.15) (end 168.31 96.15) (width 0.6) (layer "F.Cu") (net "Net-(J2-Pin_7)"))
 (segment (start 178.9 95.1) (end 175.1 98.9) (width 0.6) (layer "F.Cu") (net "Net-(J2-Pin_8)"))
 (segment (start 176.635 90.365) (end 177.5875 90.365) (width 0.6) (layer "F.Cu") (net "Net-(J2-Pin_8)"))
 (segment (start 175.1 98.9) (end 170.9 98.9) (width 0.6) (layer "F.Cu") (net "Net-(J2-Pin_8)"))
 (segment (start 175.7 82.3) (end 175.7 89.289999) (width 0.6) (layer "F.Cu") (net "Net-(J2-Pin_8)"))
 (segment (start 178.399999 90.365) (end 178.9 90.865001) (width 0.6) (layer "F.Cu") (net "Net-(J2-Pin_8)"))
 (segment (start 177.5875 90.365) (end 178.399999 90.365) (width 0.6) (layer "F.Cu") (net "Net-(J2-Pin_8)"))
 (segment (start 176 82) (end 175.7 82.3) (width 0.6) (layer "F.Cu") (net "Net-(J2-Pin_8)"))
 (segment (start 170.9 98.9) (end 169.5 97.5) (width 0.6) (layer "F.Cu") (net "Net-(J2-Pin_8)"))
 (segment (start 176.775001 90.365) (end 177.5875 90.365) (width 0.6) (layer "F.Cu") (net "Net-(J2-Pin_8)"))
 (segment (start 175.7 89.289999) (end 176.775001 90.365) (width 0.6) (layer "F.Cu") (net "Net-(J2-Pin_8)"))
 (segment (start 178.9 90.865001) (end 178.9 95.1) (width 0.6) (layer "F.Cu") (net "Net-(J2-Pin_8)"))
 (segment (start 172.04 97.5) (end 176.635 92.905) (width 0.6) (layer "F.Cu") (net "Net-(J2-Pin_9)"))
 (segment (start 176.635 92.905) (end 177.5875 92.905) (width 0.6) (layer "F.Cu") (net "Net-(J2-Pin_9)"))
 (segment (start 160.05 89.95) (end 160 90) (width 0.6) (layer "F.Cu") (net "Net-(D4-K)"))
 (segment (start 163.4 89.95) (end 160.05 89.95) (width 0.6) (layer "F.Cu") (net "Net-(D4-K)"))
 (segment (start 164.5 83.5) (end 160.35 83.5) (width 0.6) (layer "F.Cu") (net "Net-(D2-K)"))
 (segment (start 164.5 83.5) (end 168.5 83.5) (width 0.6) (layer "F.Cu") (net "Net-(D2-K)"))
 (segment (start 160.35 83.5) (end 159.2 82.35) (width 0.6) (layer "F.Cu") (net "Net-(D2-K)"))
 (segment (start 155.55 82.35) (end 159.2 82.35) (width 0.6) (layer "F.Cu") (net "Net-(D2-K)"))
 (segment (start 168.5 83.5) (end 169 83) (width 0.6) (layer "F.Cu") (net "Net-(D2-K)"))
 (segment (start 155 81.8) (end 155.55 82.35) (width 0.6) (layer "F.Cu") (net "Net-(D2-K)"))
 (segment (start 155 76.5) (end 155 81.8) (width 0.6) (layer "F.Cu") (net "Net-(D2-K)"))
 (segment (start 168.5 83.5) (end 168.83934 83.5) (width 0.2) (layer "F.Cu") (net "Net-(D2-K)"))
 (segment (start 173.9 81.9) (end 174 82) (width 0.6) (layer "F.Cu") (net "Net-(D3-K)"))
 (segment (start 159.61863 80.25) (end 161.26863 81.9) (width 0.6) (layer "F.Cu") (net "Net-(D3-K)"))
 (segment (start 157 76.5) (end 157 79) (width 0.6) (layer "F.Cu") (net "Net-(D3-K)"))
 (segment (start 158.25 80.25) (end 159.61863 80.25) (width 0.6) (layer "F.Cu") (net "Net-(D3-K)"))
 (segment (start 157 79) (end 158.25 80.25) (width 0.6) (layer "F.Cu") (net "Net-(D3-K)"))
 (segment (start 173.35 82.65) (end 174 82) (width 0.6) (layer "F.Cu") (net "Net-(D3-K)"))
 (segment (start 161.26863 81.9) (end 173.9 81.9) (width 0.6) (layer "F.Cu") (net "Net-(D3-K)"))
 (segment (start 173.35 85) (end 173.35 82.65) (width 0.6) (layer "F.Cu") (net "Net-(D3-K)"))
 (segment (start 152.5 76) (end 152.5 81.75) (width 0.6) (layer "F.Cu") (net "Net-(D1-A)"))
 (segment (start 152.5 81.75) (end 152 82.25) (width 0.6) (layer "F.Cu") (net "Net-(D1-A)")))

